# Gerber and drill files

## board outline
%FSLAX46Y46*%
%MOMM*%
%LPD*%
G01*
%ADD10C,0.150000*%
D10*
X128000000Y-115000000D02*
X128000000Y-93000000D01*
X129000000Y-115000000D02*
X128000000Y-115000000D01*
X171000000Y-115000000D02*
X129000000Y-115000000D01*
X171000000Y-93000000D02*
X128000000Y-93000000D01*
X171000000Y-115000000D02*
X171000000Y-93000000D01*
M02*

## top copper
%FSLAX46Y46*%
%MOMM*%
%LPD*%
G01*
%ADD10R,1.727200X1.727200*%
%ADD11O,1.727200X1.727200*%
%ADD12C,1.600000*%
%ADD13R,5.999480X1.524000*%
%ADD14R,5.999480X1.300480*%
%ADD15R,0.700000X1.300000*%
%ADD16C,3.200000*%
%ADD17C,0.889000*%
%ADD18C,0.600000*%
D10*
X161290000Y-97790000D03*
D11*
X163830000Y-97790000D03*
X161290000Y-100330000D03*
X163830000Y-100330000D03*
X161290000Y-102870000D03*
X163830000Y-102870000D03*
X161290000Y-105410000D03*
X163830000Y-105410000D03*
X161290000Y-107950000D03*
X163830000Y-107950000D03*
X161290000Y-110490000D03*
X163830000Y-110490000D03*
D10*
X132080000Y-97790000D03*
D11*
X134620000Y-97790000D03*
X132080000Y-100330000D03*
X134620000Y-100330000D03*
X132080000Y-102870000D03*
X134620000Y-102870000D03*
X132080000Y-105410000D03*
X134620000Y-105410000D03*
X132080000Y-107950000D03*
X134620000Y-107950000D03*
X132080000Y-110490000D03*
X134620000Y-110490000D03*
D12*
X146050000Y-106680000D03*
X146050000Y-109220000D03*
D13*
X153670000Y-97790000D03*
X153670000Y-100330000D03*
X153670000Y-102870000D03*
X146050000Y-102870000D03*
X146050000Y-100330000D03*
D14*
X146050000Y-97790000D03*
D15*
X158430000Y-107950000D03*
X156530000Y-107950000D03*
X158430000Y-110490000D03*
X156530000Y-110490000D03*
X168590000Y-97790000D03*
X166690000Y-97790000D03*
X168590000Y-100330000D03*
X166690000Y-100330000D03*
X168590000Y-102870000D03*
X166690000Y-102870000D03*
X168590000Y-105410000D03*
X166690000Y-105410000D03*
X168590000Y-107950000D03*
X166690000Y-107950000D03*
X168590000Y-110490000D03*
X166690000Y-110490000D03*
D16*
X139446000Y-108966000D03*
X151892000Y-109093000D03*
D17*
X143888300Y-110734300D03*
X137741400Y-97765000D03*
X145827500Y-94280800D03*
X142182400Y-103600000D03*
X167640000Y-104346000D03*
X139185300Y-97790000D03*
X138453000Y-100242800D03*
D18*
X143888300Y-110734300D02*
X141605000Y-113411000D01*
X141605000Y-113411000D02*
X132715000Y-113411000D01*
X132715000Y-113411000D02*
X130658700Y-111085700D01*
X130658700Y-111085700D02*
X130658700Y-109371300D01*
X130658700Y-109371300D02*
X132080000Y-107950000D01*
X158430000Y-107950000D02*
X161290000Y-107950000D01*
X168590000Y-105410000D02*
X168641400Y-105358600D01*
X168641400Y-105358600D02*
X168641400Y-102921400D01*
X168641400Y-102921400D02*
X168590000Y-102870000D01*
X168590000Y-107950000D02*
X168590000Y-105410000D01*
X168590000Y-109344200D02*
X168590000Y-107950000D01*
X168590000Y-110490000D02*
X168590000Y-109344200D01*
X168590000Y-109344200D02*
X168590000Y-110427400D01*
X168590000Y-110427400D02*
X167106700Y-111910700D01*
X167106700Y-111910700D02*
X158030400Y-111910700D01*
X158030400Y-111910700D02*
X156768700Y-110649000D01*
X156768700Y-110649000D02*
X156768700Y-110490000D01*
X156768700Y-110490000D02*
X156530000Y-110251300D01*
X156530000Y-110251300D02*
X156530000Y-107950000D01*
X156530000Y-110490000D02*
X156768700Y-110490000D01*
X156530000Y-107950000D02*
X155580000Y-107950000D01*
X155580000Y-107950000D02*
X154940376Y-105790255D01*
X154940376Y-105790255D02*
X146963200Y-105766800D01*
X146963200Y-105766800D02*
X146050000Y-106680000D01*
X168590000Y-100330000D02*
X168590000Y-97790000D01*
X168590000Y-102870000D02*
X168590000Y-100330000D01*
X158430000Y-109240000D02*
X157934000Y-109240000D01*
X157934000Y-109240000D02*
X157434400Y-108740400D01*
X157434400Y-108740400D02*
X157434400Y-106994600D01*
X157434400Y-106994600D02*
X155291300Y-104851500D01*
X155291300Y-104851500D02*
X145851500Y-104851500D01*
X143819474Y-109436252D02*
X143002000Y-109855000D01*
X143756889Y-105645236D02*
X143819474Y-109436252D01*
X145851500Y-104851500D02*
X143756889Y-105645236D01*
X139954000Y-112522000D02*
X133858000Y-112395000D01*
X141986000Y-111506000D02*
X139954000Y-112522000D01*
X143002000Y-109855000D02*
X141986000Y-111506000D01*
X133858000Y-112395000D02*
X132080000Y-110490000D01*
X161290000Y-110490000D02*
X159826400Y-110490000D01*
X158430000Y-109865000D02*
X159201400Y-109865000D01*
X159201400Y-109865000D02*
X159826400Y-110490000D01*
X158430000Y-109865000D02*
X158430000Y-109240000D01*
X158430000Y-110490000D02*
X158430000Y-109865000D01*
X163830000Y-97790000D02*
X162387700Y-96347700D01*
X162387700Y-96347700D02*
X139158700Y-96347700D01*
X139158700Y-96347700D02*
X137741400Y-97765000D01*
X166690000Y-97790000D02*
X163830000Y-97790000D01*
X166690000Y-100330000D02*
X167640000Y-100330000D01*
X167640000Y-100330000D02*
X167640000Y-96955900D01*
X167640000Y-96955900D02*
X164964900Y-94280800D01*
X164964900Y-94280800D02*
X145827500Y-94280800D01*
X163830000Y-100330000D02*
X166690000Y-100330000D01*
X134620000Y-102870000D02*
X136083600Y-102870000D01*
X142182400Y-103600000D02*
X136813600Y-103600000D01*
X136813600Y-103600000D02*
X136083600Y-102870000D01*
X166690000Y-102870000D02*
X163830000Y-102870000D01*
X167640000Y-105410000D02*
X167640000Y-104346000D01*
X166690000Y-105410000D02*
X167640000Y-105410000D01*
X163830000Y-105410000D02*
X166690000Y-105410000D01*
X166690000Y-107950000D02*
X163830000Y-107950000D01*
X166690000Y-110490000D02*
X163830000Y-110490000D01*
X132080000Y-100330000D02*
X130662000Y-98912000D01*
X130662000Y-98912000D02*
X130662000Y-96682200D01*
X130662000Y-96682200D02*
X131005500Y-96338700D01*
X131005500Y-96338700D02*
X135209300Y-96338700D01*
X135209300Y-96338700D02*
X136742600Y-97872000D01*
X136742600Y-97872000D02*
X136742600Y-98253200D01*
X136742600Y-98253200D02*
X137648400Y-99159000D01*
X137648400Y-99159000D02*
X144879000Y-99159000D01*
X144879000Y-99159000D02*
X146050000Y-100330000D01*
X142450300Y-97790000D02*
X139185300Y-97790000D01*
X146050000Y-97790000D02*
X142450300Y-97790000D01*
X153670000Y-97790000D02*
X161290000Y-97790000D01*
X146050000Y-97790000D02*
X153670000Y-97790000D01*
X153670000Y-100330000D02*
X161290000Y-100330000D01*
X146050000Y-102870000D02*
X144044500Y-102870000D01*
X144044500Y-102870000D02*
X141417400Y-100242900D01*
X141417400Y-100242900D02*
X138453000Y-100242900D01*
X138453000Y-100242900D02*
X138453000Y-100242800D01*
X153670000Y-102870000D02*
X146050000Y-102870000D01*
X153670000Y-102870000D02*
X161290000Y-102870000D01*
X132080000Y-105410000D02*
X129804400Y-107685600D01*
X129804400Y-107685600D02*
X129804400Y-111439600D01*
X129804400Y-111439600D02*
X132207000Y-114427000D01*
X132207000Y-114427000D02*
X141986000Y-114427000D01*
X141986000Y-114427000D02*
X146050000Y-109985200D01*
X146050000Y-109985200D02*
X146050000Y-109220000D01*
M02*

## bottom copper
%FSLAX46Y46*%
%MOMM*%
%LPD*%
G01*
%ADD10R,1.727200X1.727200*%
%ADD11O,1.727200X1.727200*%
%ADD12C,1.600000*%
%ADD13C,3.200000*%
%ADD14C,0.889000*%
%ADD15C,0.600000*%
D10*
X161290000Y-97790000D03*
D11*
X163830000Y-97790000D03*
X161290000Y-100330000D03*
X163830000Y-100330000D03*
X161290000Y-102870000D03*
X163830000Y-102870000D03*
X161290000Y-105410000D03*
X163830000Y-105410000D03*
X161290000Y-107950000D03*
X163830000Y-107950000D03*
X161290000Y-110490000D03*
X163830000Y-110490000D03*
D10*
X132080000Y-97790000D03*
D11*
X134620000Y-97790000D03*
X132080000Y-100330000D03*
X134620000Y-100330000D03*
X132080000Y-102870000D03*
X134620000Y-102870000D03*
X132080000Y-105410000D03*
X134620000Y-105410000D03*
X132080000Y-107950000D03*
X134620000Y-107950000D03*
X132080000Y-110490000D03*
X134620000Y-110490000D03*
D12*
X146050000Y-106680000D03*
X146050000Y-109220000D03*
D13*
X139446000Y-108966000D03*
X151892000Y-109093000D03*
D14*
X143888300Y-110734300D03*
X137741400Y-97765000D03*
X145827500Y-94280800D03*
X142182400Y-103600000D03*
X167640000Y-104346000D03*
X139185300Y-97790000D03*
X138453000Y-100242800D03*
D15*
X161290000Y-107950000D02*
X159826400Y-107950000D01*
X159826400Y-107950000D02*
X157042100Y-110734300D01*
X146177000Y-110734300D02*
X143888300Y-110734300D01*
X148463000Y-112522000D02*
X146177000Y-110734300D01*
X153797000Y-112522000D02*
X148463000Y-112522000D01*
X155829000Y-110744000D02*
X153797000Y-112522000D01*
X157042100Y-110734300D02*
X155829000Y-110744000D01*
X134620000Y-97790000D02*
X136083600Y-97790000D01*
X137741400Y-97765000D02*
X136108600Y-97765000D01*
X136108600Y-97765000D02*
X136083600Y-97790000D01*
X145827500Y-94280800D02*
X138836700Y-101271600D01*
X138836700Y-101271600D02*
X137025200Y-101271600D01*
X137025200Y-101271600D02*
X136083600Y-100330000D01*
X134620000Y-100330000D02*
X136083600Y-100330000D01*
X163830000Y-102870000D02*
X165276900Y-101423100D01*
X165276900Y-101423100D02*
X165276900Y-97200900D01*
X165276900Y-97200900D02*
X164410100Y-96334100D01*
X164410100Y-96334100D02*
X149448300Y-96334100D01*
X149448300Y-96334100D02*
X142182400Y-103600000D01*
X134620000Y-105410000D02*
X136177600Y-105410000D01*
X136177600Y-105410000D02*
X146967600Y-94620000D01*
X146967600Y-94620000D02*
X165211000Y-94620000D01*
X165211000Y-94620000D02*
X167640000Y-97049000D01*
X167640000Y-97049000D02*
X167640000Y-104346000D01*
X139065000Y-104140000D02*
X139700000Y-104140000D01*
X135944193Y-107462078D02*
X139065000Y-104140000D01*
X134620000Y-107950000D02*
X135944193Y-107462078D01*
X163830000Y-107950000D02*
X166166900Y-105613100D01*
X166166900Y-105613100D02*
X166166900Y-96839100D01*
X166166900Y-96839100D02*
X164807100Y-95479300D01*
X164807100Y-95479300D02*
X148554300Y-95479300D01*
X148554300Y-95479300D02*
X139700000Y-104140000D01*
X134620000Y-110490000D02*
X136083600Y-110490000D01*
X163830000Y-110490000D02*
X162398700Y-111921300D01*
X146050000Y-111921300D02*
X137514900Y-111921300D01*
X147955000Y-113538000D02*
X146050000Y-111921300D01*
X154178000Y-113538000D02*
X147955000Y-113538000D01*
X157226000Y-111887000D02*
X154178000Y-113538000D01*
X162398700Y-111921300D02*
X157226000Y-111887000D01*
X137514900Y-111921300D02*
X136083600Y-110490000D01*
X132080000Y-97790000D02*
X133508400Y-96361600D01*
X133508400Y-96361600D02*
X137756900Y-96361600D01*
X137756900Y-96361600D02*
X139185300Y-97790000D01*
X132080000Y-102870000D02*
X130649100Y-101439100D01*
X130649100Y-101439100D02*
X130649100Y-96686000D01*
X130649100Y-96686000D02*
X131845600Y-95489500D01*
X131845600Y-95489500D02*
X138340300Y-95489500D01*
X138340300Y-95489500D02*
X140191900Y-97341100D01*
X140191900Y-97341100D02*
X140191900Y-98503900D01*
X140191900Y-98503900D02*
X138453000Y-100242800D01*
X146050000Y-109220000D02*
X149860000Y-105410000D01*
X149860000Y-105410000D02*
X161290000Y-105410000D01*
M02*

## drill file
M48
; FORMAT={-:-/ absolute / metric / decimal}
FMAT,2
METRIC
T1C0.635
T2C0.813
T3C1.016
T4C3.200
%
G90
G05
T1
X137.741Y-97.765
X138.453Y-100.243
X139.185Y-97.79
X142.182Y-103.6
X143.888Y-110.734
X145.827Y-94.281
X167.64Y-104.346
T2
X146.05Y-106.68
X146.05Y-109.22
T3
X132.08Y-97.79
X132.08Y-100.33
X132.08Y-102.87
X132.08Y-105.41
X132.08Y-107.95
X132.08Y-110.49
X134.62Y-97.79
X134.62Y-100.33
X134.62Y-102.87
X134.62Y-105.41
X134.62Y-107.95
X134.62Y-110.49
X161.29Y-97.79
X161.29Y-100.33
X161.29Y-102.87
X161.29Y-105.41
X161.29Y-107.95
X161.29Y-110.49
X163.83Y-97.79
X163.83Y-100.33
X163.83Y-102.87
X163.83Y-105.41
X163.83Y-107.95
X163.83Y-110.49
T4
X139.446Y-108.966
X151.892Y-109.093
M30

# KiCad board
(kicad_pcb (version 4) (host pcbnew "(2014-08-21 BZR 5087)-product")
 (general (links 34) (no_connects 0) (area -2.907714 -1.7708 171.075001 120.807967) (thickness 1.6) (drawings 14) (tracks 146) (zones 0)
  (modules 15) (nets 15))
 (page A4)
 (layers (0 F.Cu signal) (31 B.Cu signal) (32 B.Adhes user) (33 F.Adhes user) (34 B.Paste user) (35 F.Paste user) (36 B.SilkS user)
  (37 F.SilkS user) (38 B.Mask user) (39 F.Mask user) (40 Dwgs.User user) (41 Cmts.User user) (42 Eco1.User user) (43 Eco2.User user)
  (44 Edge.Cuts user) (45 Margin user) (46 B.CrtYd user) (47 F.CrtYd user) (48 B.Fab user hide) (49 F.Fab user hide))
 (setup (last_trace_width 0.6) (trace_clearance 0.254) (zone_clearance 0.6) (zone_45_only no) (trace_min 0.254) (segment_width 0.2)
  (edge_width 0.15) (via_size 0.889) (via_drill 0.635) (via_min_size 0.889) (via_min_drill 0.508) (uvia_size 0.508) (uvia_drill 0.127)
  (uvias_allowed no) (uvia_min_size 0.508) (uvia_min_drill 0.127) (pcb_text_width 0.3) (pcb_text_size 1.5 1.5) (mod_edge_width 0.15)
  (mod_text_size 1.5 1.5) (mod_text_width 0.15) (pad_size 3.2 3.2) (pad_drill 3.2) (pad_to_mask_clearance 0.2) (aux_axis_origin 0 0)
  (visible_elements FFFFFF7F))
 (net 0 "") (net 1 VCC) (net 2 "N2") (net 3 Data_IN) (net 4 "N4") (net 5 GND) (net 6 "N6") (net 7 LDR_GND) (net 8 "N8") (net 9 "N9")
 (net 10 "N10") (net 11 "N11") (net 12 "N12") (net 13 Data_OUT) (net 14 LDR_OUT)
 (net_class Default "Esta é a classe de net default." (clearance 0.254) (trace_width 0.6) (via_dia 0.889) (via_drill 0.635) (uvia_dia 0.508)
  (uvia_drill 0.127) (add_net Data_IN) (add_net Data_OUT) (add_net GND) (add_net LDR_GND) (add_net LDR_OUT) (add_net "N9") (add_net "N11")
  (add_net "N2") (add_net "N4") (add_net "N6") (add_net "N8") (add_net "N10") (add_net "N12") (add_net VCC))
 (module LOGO (layer F.Cu) (at 0 0)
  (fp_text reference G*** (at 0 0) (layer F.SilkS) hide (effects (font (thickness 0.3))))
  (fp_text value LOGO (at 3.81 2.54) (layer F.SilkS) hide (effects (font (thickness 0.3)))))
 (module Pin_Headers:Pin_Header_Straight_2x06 (layer F.Cu) (at 161.29 97.79)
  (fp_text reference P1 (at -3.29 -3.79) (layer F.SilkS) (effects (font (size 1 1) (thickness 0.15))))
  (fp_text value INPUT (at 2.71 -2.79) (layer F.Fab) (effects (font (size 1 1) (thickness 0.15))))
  (pad 1 thru_hole rect (at 0 0) (size 1.7272 1.7272) (drill 1.016) (layers *.Cu *.Mask F.SilkS) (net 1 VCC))
  (pad 2 thru_hole oval (at 2.54 0) (size 1.7272 1.7272) (drill 1.016) (layers *.Cu *.Mask F.SilkS) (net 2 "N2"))
  (pad 3 thru_hole oval (at 0 2.54) (size 1.7272 1.7272) (drill 1.016) (layers *.Cu *.Mask F.SilkS) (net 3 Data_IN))
  (pad 4 thru_hole oval (at 2.54 2.54) (size 1.7272 1.7272) (drill 1.016) (layers *.Cu *.Mask F.SilkS) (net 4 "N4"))
  (pad 5 thru_hole oval (at 0 5.08) (size 1.7272 1.7272) (drill 1.016) (layers *.Cu *.Mask F.SilkS) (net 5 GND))
  (pad 6 thru_hole oval (at 2.54 5.08) (size 1.7272 1.7272) (drill 1.016) (layers *.Cu *.Mask F.SilkS) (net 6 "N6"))
  (pad 7 thru_hole oval (at 0 7.62) (size 1.7272 1.7272) (drill 1.016) (layers *.Cu *.Mask F.SilkS) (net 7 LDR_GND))
  (pad 8 thru_hole oval (at 2.54 7.62) (size 1.7272 1.7272) (drill 1.016) (layers *.Cu *.Mask F.SilkS) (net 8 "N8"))
  (pad 9 thru_hole oval (at 0 10.16) (size 1.7272 1.7272) (drill 1.016) (layers *.Cu *.Mask F.SilkS) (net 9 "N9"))
  (pad 10 thru_hole oval (at 2.54 10.16) (size 1.7272 1.7272) (drill 1.016) (layers *.Cu *.Mask F.SilkS) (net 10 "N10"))
  (pad 11 thru_hole oval (at 0 12.7) (size 1.7272 1.7272) (drill 1.016) (layers *.Cu *.Mask F.SilkS) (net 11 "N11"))
  (pad 12 thru_hole oval (at 2.54 12.7) (size 1.7272 1.7272) (drill 1.016) (layers *.Cu *.Mask F.SilkS) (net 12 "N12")))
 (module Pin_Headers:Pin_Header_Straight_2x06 (layer F.Cu) (at 132.08 97.79)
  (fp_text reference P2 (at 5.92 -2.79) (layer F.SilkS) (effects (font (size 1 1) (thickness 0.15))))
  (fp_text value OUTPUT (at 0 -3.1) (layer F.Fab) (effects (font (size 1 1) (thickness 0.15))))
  (pad 1 thru_hole rect (at 0 0) (size 1.7272 1.7272) (drill 1.016) (layers *.Cu *.Mask F.SilkS) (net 1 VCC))
  (pad 2 thru_hole oval (at 2.54 0) (size 1.7272 1.7272) (drill 1.016) (layers *.Cu *.Mask F.SilkS) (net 2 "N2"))
  (pad 3 thru_hole oval (at 0 2.54) (size 1.7272 1.7272) (drill 1.016) (layers *.Cu *.Mask F.SilkS) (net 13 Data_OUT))
  (pad 4 thru_hole oval (at 2.54 2.54) (size 1.7272 1.7272) (drill 1.016) (layers *.Cu *.Mask F.SilkS) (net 4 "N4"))
  (pad 5 thru_hole oval (at 0 5.08) (size 1.7272 1.7272) (drill 1.016) (layers *.Cu *.Mask F.SilkS) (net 5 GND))
  (pad 6 thru_hole oval (at 2.54 5.08) (size 1.7272 1.7272) (drill 1.016) (layers *.Cu *.Mask F.SilkS) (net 6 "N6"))
  (pad 7 thru_hole oval (at 0 7.62) (size 1.7272 1.7272) (drill 1.016) (layers *.Cu *.Mask F.SilkS) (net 7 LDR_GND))
  (pad 8 thru_hole oval (at 2.54 7.62) (size 1.7272 1.7272) (drill 1.016) (layers *.Cu *.Mask F.SilkS) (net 8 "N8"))
  (pad 9 thru_hole oval (at 0 10.16) (size 1.7272 1.7272) (drill 1.016) (layers *.Cu *.Mask F.SilkS) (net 9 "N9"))
  (pad 10 thru_hole oval (at 2.54 10.16) (size 1.7272 1.7272) (drill 1.016) (layers *.Cu *.Mask F.SilkS) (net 10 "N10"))
  (pad 11 thru_hole oval (at 0 12.7) (size 1.7272 1.7272) (drill 1.016) (layers *.Cu *.Mask F.SilkS) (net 11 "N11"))
  (pad 12 thru_hole oval (at 2.54 12.7) (size 1.7272 1.7272) (drill 1.016) (layers *.Cu *.Mask F.SilkS) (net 12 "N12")))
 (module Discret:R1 (layer F.Cu) (at 146.05 107.95 270)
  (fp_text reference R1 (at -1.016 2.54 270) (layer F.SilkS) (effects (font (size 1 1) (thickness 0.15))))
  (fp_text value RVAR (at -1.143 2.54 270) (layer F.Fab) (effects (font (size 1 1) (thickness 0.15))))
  (pad 1 thru_hole circle (at -1.27 0 270) (size 1.6 1.6) (drill 0.8128) (layers *.Cu *.Mask F.SilkS) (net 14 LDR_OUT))
  (pad 2 thru_hole circle (at 1.27 0 270) (size 1.6 1.6) (drill 0.8128) (layers *.Cu *.Mask F.SilkS) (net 7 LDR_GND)))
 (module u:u (layer F.Cu) (at 149.86 100.33)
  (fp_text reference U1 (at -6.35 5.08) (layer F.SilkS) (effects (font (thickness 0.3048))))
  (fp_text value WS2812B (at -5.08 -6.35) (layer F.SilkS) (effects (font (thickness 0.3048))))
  (pad 1 smd rect (at 3.81 -2.54) (size 5.99948 1.524) (layers F.Cu F.Paste F.Mask) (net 1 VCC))
  (pad 2 smd rect (at 3.81 0) (size 5.99948 1.524) (layers F.Cu F.Paste F.Mask) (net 3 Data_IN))
  (pad 3 smd rect (at 3.81 2.54) (size 5.99948 1.524) (layers F.Cu F.Paste F.Mask) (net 5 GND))
  (pad 4 smd rect (at -3.81 2.54) (size 5.99948 1.524) (layers F.Cu F.Paste F.Mask) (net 5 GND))
  (pad 5 smd rect (at -3.81 0) (size 5.99948 1.524) (layers F.Cu F.Paste F.Mask) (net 13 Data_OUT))
  (pad 6 smd rect (at -3.81 -2.54) (size 5.99948 1.30048) (layers F.Cu F.Paste F.Mask) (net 1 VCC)))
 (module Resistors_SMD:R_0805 (layer F.Cu) (at 157.48 107.95 180)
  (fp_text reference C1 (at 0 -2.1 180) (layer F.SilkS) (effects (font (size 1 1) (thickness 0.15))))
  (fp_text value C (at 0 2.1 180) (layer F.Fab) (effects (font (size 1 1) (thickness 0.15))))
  (pad 1 smd rect (at -0.95 0 180) (size 0.7 1.3) (layers F.Cu F.Paste F.Mask) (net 9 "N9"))
  (pad 2 smd rect (at 0.95 0 180) (size 0.7 1.3) (layers F.Cu F.Paste F.Mask) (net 14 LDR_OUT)))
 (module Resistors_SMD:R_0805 (layer F.Cu) (at 157.48 110.49 180)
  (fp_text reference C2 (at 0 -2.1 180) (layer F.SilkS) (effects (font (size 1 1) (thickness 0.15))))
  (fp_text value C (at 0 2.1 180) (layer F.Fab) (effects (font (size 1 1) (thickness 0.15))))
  (pad 1 smd rect (at -0.95 0 180) (size 0.7 1.3) (layers F.Cu F.Paste F.Mask) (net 11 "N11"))
  (pad 2 smd rect (at 0.95 0 180) (size 0.7 1.3) (layers F.Cu F.Paste F.Mask) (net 14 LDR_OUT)))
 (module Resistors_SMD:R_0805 (layer F.Cu) (at 167.64 97.79 180)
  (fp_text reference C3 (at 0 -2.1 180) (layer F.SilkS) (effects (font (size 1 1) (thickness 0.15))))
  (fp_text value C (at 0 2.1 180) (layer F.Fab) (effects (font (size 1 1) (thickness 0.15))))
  (pad 1 smd rect (at -0.95 0 180) (size 0.7 1.3) (layers F.Cu F.Paste F.Mask) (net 14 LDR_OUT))
  (pad 2 smd rect (at 0.95 0 180) (size 0.7 1.3) (layers F.Cu F.Paste F.Mask) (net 2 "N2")))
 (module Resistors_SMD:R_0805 (layer F.Cu) (at 167.64 100.33 180)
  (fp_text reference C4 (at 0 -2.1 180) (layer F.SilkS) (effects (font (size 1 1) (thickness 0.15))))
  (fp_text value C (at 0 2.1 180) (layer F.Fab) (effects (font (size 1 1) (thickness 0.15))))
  (pad 1 smd rect (at -0.95 0 180) (size 0.7 1.3) (layers F.Cu F.Paste F.Mask) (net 14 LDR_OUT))
  (pad 2 smd rect (at 0.95 0 180) (size 0.7 1.3) (layers F.Cu F.Paste F.Mask) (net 4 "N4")))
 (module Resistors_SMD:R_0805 (layer F.Cu) (at 167.64 102.87 180)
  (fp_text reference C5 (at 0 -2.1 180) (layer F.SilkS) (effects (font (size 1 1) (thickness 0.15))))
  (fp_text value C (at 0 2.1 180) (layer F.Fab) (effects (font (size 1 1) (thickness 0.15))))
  (pad 1 smd rect (at -0.95 0 180) (size 0.7 1.3) (layers F.Cu F.Paste F.Mask) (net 14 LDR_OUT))
  (pad 2 smd rect (at 0.95 0 180) (size 0.7 1.3) (layers F.Cu F.Paste F.Mask) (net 6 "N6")))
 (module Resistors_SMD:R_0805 (layer F.Cu) (at 167.64 105.41 180)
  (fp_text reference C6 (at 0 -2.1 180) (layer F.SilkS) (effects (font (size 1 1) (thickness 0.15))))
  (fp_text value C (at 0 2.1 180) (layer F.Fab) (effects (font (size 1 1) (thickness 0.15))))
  (pad 1 smd rect (at -0.95 0 180) (size 0.7 1.3) (layers F.Cu F.Paste F.Mask) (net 14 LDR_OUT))
  (pad 2 smd rect (at 0.95 0 180) (size 0.7 1.3) (layers F.Cu F.Paste F.Mask) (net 8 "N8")))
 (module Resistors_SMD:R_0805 (layer F.Cu) (at 167.64 107.95 180)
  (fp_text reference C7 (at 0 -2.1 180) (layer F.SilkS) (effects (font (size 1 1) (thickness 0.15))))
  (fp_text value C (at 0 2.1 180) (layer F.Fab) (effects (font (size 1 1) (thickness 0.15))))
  (pad 1 smd rect (at -0.95 0 180) (size 0.7 1.3) (layers F.Cu F.Paste F.Mask) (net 14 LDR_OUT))
  (pad 2 smd rect (at 0.95 0 180) (size 0.7 1.3) (layers F.Cu F.Paste F.Mask) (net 10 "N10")))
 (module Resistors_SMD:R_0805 (layer F.Cu) (at 167.64 110.49 180)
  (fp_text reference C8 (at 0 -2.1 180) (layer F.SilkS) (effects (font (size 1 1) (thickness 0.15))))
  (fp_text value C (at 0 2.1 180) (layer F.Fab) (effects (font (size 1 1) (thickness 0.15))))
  (pad 1 smd rect (at -0.95 0 180) (size 0.7 1.3) (layers F.Cu F.Paste F.Mask) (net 14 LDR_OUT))
  (pad 2 smd rect (at 0.95 0 180) (size 0.7 1.3) (layers F.Cu F.Paste F.Mask) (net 12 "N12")))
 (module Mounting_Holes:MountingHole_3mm (layer F.Cu) (at 139.446 108.966)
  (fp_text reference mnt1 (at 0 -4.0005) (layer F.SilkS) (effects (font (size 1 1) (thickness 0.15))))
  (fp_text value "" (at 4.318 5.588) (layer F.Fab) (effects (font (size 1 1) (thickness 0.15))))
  (pad "" thru_hole circle (at 0 0) (size 3.2 3.2) (drill 3.2) (layers *.Cu *.Mask F.SilkS)))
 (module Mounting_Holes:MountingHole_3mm (layer F.Cu) (at 151.892 109.093)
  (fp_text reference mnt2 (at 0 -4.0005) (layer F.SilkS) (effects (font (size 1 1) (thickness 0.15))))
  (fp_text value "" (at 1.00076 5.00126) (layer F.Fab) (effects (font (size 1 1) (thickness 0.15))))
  (pad "" thru_hole circle (at 0 0) (size 3.2 3.2) (drill 3.2) (layers *.Cu)))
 (gr_line (start 128 115) (end 128 93) (angle 90) (layer Edge.Cuts) (width 0.15))
 (gr_line (start 129 115) (end 128 115) (angle 90) (layer Edge.Cuts) (width 0.15))
 (gr_line (start 171 115) (end 129 115) (angle 90) (layer Edge.Cuts) (width 0.15))
 (gr_line (start 171 93) (end 128 93) (angle 90) (layer Edge.Cuts) (width 0.15))
 (gr_line (start 171 115) (end 171 93) (angle 90) (layer Edge.Cuts) (width 0.15))
 (segment (start 161.29 107.95) (end 159.8264 107.95) (width 0.6) (layer B.Cu) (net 9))
 (segment (start 143.8883 110.7343) (end 141.605 113.411) (width 0.6) (layer F.Cu) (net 9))
 (segment (start 141.605 113.411) (end 132.715 113.411) (width 0.6) (layer F.Cu) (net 9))
 (segment (start 132.715 113.411) (end 130.6587 111.0857) (width 0.6) (layer F.Cu) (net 9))
 (segment (start 130.6587 111.0857) (end 130.6587 109.3713) (width 0.6) (layer F.Cu) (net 9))
 (segment (start 130.6587 109.3713) (end 132.08 107.95) (width 0.6) (layer F.Cu) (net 9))
 (segment (start 159.8264 107.95) (end 157.0421 110.7343) (width 0.6) (layer B.Cu) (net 9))
 (segment (start 146.177 110.7343) (end 143.8883 110.7343) (width 0.6) (layer B.Cu) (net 9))
 (segment (start 148.463 112.522) (end 146.177 110.7343) (width 0.6) (layer B.Cu) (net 9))
 (segment (start 153.797 112.522) (end 148.463 112.522) (width 0.6) (layer B.Cu) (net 9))
 (segment (start 155.829 110.744) (end 153.797 112.522) (width 0.6) (layer B.Cu) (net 9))
 (segment (start 157.0421 110.7343) (end 155.829 110.744) (width 0.6) (layer B.Cu) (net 9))
 (segment (start 158.43 107.95) (end 161.29 107.95) (width 0.6) (layer F.Cu) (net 9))
 (via (at 143.8883 110.7343) (size 0.889) (layers F.Cu B.Cu) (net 9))
 (segment (start 168.59 105.41) (end 168.6414 105.3586) (width 0.6) (layer F.Cu) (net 14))
 (segment (start 168.6414 105.3586) (end 168.6414 102.9214) (width 0.6) (layer F.Cu) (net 14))
 (segment (start 168.6414 102.9214) (end 168.59 102.87) (width 0.6) (layer F.Cu) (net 14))
 (segment (start 168.59 107.95) (end 168.59 105.41) (width 0.6) (layer F.Cu) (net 14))
 (segment (start 168.59 109.3442) (end 168.59 107.95) (width 0.6) (layer F.Cu) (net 14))
 (segment (start 168.59 110.49) (end 168.59 109.3442) (width 0.6) (layer F.Cu) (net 14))
 (segment (start 168.59 109.3442) (end 168.59 110.4274) (width 0.6) (layer F.Cu) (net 14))
 (segment (start 168.59 110.4274) (end 167.1067 111.9107) (width 0.6) (layer F.Cu) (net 14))
 (segment (start 167.1067 111.9107) (end 158.0304 111.9107) (width 0.6) (layer F.Cu) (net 14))
 (segment (start 158.0304 111.9107) (end 156.7687 110.649) (width 0.6) (layer F.Cu) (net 14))
 (segment (start 156.7687 110.649) (end 156.7687 110.49) (width 0.6) (layer F.Cu) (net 14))
 (segment (start 156.7687 110.49) (end 156.53 110.2513) (width 0.6) (layer F.Cu) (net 14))
 (segment (start 156.53 110.2513) (end 156.53 107.95) (width 0.6) (layer F.Cu) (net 14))
 (segment (start 156.53 110.49) (end 156.7687 110.49) (width 0.6) (layer F.Cu) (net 14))
 (segment (start 156.53 107.95) (end 155.58 107.95) (width 0.6) (layer F.Cu) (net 14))
 (segment (start 155.58 107.95) (end 154.940376 105.790255) (width 0.6) (layer F.Cu) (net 14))
 (segment (start 154.940376 105.790255) (end 146.9632 105.7668) (width 0.6) (layer F.Cu) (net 14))
 (segment (start 146.9632 105.7668) (end 146.05 106.68) (width 0.6) (layer F.Cu) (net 14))
 (segment (start 168.59 100.33) (end 168.59 97.79) (width 0.6) (layer F.Cu) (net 14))
 (segment (start 168.59 102.87) (end 168.59 100.33) (width 0.6) (layer F.Cu) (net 14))
 (segment (start 158.43 109.24) (end 157.934 109.24) (width 0.6) (layer F.Cu) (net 11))
 (segment (start 157.934 109.24) (end 157.4344 108.7404) (width 0.6) (layer F.Cu) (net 11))
 (segment (start 157.4344 108.7404) (end 157.4344 106.9946) (width 0.6) (layer F.Cu) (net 11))
 (segment (start 157.4344 106.9946) (end 155.2913 104.8515) (width 0.6) (layer F.Cu) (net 11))
 (segment (start 155.2913 104.8515) (end 145.8515 104.8515) (width 0.6) (layer F.Cu) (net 11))
 (segment (start 143.819474 109.436252) (end 143.002 109.855) (width 0.6) (layer F.Cu) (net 11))
 (segment (start 143.756889 105.645236) (end 143.819474 109.436252) (width 0.6) (layer F.Cu) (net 11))
 (segment (start 145.8515 104.8515) (end 143.756889 105.645236) (width 0.6) (layer F.Cu) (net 11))
 (segment (start 139.954 112.522) (end 133.858 112.395) (width 0.6) (layer F.Cu) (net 11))
 (segment (start 141.986 111.506) (end 139.954 112.522) (width 0.6) (layer F.Cu) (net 11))
 (segment (start 143.002 109.855) (end 141.986 111.506) (width 0.6) (layer F.Cu) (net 11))
 (segment (start 133.858 112.395) (end 132.08 110.49) (width 0.6) (layer F.Cu) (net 11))
 (segment (start 161.29 110.49) (end 159.8264 110.49) (width 0.6) (layer F.Cu) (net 11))
 (segment (start 158.43 109.865) (end 159.2014 109.865) (width 0.6) (layer F.Cu) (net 11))
 (segment (start 159.2014 109.865) (end 159.8264 110.49) (width 0.6) (layer F.Cu) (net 11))
 (segment (start 158.43 109.865) (end 158.43 109.24) (width 0.6) (layer F.Cu) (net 11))
 (segment (start 158.43 110.49) (end 158.43 109.865) (width 0.6) (layer F.Cu) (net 11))
 (segment (start 163.83 97.79) (end 162.3877 96.3477) (width 0.6) (layer F.Cu) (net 2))
 (segment (start 162.3877 96.3477) (end 139.1587 96.3477) (width 0.6) (layer F.Cu) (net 2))
 (segment (start 139.1587 96.3477) (end 137.7414 97.765) (width 0.6) (layer F.Cu) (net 2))
 (segment (start 166.69 97.79) (end 163.83 97.79) (width 0.6) (layer F.Cu) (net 2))
 (segment (start 134.62 97.79) (end 136.0836 97.79) (width 0.6) (layer B.Cu) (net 2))
 (segment (start 137.7414 97.765) (end 136.1086 97.765) (width 0.6) (layer B.Cu) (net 2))
 (segment (start 136.1086 97.765) (end 136.0836 97.79) (width 0.6) (layer B.Cu) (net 2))
 (via (at 137.7414 97.765) (size 0.889) (layers F.Cu B.Cu) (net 2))
 (segment (start 145.8275 94.2808) (end 138.8367 101.2716) (width 0.6) (layer B.Cu) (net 4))
 (segment (start 138.8367 101.2716) (end 137.0252 101.2716) (width 0.6) (layer B.Cu) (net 4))
 (segment (start 137.0252 101.2716) (end 136.0836 100.33) (width 0.6) (layer B.Cu) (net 4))
 (segment (start 134.62 100.33) (end 136.0836 100.33) (width 0.6) (layer B.Cu) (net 4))
 (segment (start 166.69 100.33) (end 167.64 100.33) (width 0.6) (layer F.Cu) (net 4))
 (segment (start 167.64 100.33) (end 167.64 96.9559) (width 0.6) (layer F.Cu) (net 4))
 (segment (start 167.64 96.9559) (end 164.9649 94.2808) (width 0.6) (layer F.Cu) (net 4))
 (segment (start 164.9649 94.2808) (end 145.8275 94.2808) (width 0.6) (layer F.Cu) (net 4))
 (segment (start 163.83 100.33) (end 166.69 100.33) (width 0.6) (layer F.Cu) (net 4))
 (via (at 145.8275 94.2808) (size 0.889) (layers F.Cu B.Cu) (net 4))
 (segment (start 134.62 102.87) (end 136.0836 102.87) (width 0.6) (layer F.Cu) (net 6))
 (segment (start 142.1824 103.6) (end 136.8136 103.6) (width 0.6) (layer F.Cu) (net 6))
 (segment (start 136.8136 103.6) (end 136.0836 102.87) (width 0.6) (layer F.Cu) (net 6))
 (segment (start 163.83 102.87) (end 165.2769 101.4231) (width 0.6) (layer B.Cu) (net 6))
 (segment (start 165.2769 101.4231) (end 165.2769 97.2009) (width 0.6) (layer B.Cu) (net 6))
 (segment (start 165.2769 97.2009) (end 164.4101 96.3341) (width 0.6) (layer B.Cu) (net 6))
 (segment (start 164.4101 96.3341) (end 149.4483 96.3341) (width 0.6) (layer B.Cu) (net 6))
 (segment (start 149.4483 96.3341) (end 142.1824 103.6) (width 0.6) (layer B.Cu) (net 6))
 (segment (start 166.69 102.87) (end 163.83 102.87) (width 0.6) (layer F.Cu) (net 6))
 (via (at 142.1824 103.6) (size 0.889) (layers F.Cu B.Cu) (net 6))
 (segment (start 167.64 105.41) (end 167.64 104.346) (width 0.6) (layer F.Cu) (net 8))
 (segment (start 134.62 105.41) (end 136.1776 105.41) (width 0.6) (layer B.Cu) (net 8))
 (segment (start 136.1776 105.41) (end 146.9676 94.62) (width 0.6) (layer B.Cu) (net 8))
 (segment (start 146.9676 94.62) (end 165.211 94.62) (width 0.6) (layer B.Cu) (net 8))
 (segment (start 165.211 94.62) (end 167.64 97.049) (width 0.6) (layer B.Cu) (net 8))
 (segment (start 167.64 97.049) (end 167.64 104.346) (width 0.6) (layer B.Cu) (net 8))
 (segment (start 166.69 105.41) (end 167.64 105.41) (width 0.6) (layer F.Cu) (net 8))
 (segment (start 163.83 105.41) (end 166.69 105.41) (width 0.6) (layer F.Cu) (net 8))
 (via (at 167.64 104.346) (size 0.889) (layers F.Cu B.Cu) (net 8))
 (segment (start 139.065 104.14) (end 139.7 104.14) (width 0.6) (layer B.Cu) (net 10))
 (segment (start 135.944193 107.462078) (end 139.065 104.14) (width 0.6) (layer B.Cu) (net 10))
 (segment (start 134.62 107.95) (end 135.944193 107.462078) (width 0.6) (layer B.Cu) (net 10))
 (segment (start 163.83 107.95) (end 166.1669 105.6131) (width 0.6) (layer B.Cu) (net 10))
 (segment (start 166.1669 105.6131) (end 166.1669 96.8391) (width 0.6) (layer B.Cu) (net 10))
 (segment (start 166.1669 96.8391) (end 164.8071 95.4793) (width 0.6) (layer B.Cu) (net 10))
 (segment (start 164.8071 95.4793) (end 148.5543 95.4793) (width 0.6) (layer B.Cu) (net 10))
 (segment (start 148.5543 95.4793) (end 139.7 104.14) (width 0.6) (layer B.Cu) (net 10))
 (segment (start 166.69 107.95) (end 163.83 107.95) (width 0.6) (layer F.Cu) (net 10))
 (segment (start 134.62 110.49) (end 136.0836 110.49) (width 0.6) (layer B.Cu) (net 12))
 (segment (start 163.83 110.49) (end 162.3987 111.9213) (width 0.6) (layer B.Cu) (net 12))
 (segment (start 146.05 111.9213) (end 137.5149 111.9213) (width 0.6) (layer B.Cu) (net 12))
 (segment (start 147.955 113.538) (end 146.05 111.9213) (width 0.6) (layer B.Cu) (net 12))
 (segment (start 154.178 113.538) (end 147.955 113.538) (width 0.6) (layer B.Cu) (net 12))
 (segment (start 157.226 111.887) (end 154.178 113.538) (width 0.6) (layer B.Cu) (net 12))
 (segment (start 162.3987 111.9213) (end 157.226 111.887) (width 0.6) (layer B.Cu) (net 12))
 (segment (start 137.5149 111.9213) (end 136.0836 110.49) (width 0.6) (layer B.Cu) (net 12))
 (segment (start 166.69 110.49) (end 163.83 110.49) (width 0.6) (layer F.Cu) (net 12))
 (segment (start 132.08 100.33) (end 130.662 98.912) (width 0.6) (layer F.Cu) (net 13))
 (segment (start 130.662 98.912) (end 130.662 96.6822) (width 0.6) (layer F.Cu) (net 13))
 (segment (start 130.662 96.6822) (end 131.0055 96.3387) (width 0.6) (layer F.Cu) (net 13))
 (segment (start 131.0055 96.3387) (end 135.2093 96.3387) (width 0.6) (layer F.Cu) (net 13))
 (segment (start 135.2093 96.3387) (end 136.7426 97.872) (width 0.6) (layer F.Cu) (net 13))
 (segment (start 136.7426 97.872) (end 136.7426 98.2532) (width 0.6) (layer F.Cu) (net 13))
 (segment (start 136.7426 98.2532) (end 137.6484 99.159) (width 0.6) (layer F.Cu) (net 13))
 (segment (start 137.6484 99.159) (end 144.879 99.159) (width 0.6) (layer F.Cu) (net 13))
 (segment (start 144.879 99.159) (end 146.05 100.33) (width 0.6) (layer F.Cu) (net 13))
 (segment (start 142.4503 97.79) (end 139.1853 97.79) (width 0.6) (layer F.Cu) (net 1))
 (segment (start 132.08 97.79) (end 133.5084 96.3616) (width 0.6) (layer B.Cu) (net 1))
 (segment (start 133.5084 96.3616) (end 137.7569 96.3616) (width 0.6) (layer B.Cu) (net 1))
 (segment (start 137.7569 96.3616) (end 139.1853 97.79) (width 0.6) (layer B.Cu) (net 1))
 (segment (start 146.05 97.79) (end 142.4503 97.79) (width 0.6) (layer F.Cu) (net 1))
 (segment (start 153.67 97.79) (end 161.29 97.79) (width 0.6) (layer F.Cu) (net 1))
 (segment (start 146.05 97.79) (end 153.67 97.79) (width 0.6) (layer F.Cu) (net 1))
 (via (at 139.1853 97.79) (size 0.889) (layers F.Cu B.Cu) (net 1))
 (segment (start 153.67 100.33) (end 161.29 100.33) (width 0.6) (layer F.Cu) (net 3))
 (segment (start 146.05 102.87) (end 144.0445 102.87) (width 0.6) (layer F.Cu) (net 5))
 (segment (start 144.0445 102.87) (end 141.4174 100.2429) (width 0.6) (layer F.Cu) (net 5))
 (segment (start 141.4174 100.2429) (end 138.453 100.2429) (width 0.6) (layer F.Cu) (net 5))
 (segment (start 138.453 100.2429) (end 138.453 100.2428) (width 0.6) (layer F.Cu) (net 5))
 (segment (start 132.08 102.87) (end 130.6491 101.4391) (width 0.6) (layer B.Cu) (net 5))
 (segment (start 130.6491 101.4391) (end 130.6491 96.686) (width 0.6) (layer B.Cu) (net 5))
 (segment (start 130.6491 96.686) (end 131.8456 95.4895) (width 0.6) (layer B.Cu) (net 5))
 (segment (start 131.8456 95.4895) (end 138.3403 95.4895) (width 0.6) (layer B.Cu) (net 5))
 (segment (start 138.3403 95.4895) (end 140.1919 97.3411) (width 0.6) (layer B.Cu) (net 5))
 (segment (start 140.1919 97.3411) (end 140.1919 98.5039) (width 0.6) (layer B.Cu) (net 5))
 (segment (start 140.1919 98.5039) (end 138.453 100.2428) (width 0.6) (layer B.Cu) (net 5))
 (segment (start 153.67 102.87) (end 146.05 102.87) (width 0.6) (layer F.Cu) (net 5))
 (segment (start 153.67 102.87) (end 161.29 102.87) (width 0.6) (layer F.Cu) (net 5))
 (via (at 138.453 100.2428) (size 0.889) (layers F.Cu B.Cu) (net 5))
 (segment (start 132.08 105.41) (end 129.8044 107.6856) (width 0.6) (layer F.Cu) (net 7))
 (segment (start 129.8044 107.6856) (end 129.8044 111.4396) (width 0.6) (layer F.Cu) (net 7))
 (segment (start 129.8044 111.4396) (end 132.207 114.427) (width 0.6) (layer F.Cu) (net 7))
 (segment (start 132.207 114.427) (end 141.986 114.427) (width 0.6) (layer F.Cu) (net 7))
 (segment (start 141.986 114.427) (end 146.05 109.9852) (width 0.6) (layer F.Cu) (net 7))
 (segment (start 146.05 109.9852) (end 146.05 109.22) (width 0.6) (layer F.Cu) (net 7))
 (segment (start 146.05 109.22) (end 149.86 105.41) (width 0.6) (layer B.Cu) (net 7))
 (segment (start 149.86 105.41) (end 161.29 105.41) (width 0.6) (layer B.Cu) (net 7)))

